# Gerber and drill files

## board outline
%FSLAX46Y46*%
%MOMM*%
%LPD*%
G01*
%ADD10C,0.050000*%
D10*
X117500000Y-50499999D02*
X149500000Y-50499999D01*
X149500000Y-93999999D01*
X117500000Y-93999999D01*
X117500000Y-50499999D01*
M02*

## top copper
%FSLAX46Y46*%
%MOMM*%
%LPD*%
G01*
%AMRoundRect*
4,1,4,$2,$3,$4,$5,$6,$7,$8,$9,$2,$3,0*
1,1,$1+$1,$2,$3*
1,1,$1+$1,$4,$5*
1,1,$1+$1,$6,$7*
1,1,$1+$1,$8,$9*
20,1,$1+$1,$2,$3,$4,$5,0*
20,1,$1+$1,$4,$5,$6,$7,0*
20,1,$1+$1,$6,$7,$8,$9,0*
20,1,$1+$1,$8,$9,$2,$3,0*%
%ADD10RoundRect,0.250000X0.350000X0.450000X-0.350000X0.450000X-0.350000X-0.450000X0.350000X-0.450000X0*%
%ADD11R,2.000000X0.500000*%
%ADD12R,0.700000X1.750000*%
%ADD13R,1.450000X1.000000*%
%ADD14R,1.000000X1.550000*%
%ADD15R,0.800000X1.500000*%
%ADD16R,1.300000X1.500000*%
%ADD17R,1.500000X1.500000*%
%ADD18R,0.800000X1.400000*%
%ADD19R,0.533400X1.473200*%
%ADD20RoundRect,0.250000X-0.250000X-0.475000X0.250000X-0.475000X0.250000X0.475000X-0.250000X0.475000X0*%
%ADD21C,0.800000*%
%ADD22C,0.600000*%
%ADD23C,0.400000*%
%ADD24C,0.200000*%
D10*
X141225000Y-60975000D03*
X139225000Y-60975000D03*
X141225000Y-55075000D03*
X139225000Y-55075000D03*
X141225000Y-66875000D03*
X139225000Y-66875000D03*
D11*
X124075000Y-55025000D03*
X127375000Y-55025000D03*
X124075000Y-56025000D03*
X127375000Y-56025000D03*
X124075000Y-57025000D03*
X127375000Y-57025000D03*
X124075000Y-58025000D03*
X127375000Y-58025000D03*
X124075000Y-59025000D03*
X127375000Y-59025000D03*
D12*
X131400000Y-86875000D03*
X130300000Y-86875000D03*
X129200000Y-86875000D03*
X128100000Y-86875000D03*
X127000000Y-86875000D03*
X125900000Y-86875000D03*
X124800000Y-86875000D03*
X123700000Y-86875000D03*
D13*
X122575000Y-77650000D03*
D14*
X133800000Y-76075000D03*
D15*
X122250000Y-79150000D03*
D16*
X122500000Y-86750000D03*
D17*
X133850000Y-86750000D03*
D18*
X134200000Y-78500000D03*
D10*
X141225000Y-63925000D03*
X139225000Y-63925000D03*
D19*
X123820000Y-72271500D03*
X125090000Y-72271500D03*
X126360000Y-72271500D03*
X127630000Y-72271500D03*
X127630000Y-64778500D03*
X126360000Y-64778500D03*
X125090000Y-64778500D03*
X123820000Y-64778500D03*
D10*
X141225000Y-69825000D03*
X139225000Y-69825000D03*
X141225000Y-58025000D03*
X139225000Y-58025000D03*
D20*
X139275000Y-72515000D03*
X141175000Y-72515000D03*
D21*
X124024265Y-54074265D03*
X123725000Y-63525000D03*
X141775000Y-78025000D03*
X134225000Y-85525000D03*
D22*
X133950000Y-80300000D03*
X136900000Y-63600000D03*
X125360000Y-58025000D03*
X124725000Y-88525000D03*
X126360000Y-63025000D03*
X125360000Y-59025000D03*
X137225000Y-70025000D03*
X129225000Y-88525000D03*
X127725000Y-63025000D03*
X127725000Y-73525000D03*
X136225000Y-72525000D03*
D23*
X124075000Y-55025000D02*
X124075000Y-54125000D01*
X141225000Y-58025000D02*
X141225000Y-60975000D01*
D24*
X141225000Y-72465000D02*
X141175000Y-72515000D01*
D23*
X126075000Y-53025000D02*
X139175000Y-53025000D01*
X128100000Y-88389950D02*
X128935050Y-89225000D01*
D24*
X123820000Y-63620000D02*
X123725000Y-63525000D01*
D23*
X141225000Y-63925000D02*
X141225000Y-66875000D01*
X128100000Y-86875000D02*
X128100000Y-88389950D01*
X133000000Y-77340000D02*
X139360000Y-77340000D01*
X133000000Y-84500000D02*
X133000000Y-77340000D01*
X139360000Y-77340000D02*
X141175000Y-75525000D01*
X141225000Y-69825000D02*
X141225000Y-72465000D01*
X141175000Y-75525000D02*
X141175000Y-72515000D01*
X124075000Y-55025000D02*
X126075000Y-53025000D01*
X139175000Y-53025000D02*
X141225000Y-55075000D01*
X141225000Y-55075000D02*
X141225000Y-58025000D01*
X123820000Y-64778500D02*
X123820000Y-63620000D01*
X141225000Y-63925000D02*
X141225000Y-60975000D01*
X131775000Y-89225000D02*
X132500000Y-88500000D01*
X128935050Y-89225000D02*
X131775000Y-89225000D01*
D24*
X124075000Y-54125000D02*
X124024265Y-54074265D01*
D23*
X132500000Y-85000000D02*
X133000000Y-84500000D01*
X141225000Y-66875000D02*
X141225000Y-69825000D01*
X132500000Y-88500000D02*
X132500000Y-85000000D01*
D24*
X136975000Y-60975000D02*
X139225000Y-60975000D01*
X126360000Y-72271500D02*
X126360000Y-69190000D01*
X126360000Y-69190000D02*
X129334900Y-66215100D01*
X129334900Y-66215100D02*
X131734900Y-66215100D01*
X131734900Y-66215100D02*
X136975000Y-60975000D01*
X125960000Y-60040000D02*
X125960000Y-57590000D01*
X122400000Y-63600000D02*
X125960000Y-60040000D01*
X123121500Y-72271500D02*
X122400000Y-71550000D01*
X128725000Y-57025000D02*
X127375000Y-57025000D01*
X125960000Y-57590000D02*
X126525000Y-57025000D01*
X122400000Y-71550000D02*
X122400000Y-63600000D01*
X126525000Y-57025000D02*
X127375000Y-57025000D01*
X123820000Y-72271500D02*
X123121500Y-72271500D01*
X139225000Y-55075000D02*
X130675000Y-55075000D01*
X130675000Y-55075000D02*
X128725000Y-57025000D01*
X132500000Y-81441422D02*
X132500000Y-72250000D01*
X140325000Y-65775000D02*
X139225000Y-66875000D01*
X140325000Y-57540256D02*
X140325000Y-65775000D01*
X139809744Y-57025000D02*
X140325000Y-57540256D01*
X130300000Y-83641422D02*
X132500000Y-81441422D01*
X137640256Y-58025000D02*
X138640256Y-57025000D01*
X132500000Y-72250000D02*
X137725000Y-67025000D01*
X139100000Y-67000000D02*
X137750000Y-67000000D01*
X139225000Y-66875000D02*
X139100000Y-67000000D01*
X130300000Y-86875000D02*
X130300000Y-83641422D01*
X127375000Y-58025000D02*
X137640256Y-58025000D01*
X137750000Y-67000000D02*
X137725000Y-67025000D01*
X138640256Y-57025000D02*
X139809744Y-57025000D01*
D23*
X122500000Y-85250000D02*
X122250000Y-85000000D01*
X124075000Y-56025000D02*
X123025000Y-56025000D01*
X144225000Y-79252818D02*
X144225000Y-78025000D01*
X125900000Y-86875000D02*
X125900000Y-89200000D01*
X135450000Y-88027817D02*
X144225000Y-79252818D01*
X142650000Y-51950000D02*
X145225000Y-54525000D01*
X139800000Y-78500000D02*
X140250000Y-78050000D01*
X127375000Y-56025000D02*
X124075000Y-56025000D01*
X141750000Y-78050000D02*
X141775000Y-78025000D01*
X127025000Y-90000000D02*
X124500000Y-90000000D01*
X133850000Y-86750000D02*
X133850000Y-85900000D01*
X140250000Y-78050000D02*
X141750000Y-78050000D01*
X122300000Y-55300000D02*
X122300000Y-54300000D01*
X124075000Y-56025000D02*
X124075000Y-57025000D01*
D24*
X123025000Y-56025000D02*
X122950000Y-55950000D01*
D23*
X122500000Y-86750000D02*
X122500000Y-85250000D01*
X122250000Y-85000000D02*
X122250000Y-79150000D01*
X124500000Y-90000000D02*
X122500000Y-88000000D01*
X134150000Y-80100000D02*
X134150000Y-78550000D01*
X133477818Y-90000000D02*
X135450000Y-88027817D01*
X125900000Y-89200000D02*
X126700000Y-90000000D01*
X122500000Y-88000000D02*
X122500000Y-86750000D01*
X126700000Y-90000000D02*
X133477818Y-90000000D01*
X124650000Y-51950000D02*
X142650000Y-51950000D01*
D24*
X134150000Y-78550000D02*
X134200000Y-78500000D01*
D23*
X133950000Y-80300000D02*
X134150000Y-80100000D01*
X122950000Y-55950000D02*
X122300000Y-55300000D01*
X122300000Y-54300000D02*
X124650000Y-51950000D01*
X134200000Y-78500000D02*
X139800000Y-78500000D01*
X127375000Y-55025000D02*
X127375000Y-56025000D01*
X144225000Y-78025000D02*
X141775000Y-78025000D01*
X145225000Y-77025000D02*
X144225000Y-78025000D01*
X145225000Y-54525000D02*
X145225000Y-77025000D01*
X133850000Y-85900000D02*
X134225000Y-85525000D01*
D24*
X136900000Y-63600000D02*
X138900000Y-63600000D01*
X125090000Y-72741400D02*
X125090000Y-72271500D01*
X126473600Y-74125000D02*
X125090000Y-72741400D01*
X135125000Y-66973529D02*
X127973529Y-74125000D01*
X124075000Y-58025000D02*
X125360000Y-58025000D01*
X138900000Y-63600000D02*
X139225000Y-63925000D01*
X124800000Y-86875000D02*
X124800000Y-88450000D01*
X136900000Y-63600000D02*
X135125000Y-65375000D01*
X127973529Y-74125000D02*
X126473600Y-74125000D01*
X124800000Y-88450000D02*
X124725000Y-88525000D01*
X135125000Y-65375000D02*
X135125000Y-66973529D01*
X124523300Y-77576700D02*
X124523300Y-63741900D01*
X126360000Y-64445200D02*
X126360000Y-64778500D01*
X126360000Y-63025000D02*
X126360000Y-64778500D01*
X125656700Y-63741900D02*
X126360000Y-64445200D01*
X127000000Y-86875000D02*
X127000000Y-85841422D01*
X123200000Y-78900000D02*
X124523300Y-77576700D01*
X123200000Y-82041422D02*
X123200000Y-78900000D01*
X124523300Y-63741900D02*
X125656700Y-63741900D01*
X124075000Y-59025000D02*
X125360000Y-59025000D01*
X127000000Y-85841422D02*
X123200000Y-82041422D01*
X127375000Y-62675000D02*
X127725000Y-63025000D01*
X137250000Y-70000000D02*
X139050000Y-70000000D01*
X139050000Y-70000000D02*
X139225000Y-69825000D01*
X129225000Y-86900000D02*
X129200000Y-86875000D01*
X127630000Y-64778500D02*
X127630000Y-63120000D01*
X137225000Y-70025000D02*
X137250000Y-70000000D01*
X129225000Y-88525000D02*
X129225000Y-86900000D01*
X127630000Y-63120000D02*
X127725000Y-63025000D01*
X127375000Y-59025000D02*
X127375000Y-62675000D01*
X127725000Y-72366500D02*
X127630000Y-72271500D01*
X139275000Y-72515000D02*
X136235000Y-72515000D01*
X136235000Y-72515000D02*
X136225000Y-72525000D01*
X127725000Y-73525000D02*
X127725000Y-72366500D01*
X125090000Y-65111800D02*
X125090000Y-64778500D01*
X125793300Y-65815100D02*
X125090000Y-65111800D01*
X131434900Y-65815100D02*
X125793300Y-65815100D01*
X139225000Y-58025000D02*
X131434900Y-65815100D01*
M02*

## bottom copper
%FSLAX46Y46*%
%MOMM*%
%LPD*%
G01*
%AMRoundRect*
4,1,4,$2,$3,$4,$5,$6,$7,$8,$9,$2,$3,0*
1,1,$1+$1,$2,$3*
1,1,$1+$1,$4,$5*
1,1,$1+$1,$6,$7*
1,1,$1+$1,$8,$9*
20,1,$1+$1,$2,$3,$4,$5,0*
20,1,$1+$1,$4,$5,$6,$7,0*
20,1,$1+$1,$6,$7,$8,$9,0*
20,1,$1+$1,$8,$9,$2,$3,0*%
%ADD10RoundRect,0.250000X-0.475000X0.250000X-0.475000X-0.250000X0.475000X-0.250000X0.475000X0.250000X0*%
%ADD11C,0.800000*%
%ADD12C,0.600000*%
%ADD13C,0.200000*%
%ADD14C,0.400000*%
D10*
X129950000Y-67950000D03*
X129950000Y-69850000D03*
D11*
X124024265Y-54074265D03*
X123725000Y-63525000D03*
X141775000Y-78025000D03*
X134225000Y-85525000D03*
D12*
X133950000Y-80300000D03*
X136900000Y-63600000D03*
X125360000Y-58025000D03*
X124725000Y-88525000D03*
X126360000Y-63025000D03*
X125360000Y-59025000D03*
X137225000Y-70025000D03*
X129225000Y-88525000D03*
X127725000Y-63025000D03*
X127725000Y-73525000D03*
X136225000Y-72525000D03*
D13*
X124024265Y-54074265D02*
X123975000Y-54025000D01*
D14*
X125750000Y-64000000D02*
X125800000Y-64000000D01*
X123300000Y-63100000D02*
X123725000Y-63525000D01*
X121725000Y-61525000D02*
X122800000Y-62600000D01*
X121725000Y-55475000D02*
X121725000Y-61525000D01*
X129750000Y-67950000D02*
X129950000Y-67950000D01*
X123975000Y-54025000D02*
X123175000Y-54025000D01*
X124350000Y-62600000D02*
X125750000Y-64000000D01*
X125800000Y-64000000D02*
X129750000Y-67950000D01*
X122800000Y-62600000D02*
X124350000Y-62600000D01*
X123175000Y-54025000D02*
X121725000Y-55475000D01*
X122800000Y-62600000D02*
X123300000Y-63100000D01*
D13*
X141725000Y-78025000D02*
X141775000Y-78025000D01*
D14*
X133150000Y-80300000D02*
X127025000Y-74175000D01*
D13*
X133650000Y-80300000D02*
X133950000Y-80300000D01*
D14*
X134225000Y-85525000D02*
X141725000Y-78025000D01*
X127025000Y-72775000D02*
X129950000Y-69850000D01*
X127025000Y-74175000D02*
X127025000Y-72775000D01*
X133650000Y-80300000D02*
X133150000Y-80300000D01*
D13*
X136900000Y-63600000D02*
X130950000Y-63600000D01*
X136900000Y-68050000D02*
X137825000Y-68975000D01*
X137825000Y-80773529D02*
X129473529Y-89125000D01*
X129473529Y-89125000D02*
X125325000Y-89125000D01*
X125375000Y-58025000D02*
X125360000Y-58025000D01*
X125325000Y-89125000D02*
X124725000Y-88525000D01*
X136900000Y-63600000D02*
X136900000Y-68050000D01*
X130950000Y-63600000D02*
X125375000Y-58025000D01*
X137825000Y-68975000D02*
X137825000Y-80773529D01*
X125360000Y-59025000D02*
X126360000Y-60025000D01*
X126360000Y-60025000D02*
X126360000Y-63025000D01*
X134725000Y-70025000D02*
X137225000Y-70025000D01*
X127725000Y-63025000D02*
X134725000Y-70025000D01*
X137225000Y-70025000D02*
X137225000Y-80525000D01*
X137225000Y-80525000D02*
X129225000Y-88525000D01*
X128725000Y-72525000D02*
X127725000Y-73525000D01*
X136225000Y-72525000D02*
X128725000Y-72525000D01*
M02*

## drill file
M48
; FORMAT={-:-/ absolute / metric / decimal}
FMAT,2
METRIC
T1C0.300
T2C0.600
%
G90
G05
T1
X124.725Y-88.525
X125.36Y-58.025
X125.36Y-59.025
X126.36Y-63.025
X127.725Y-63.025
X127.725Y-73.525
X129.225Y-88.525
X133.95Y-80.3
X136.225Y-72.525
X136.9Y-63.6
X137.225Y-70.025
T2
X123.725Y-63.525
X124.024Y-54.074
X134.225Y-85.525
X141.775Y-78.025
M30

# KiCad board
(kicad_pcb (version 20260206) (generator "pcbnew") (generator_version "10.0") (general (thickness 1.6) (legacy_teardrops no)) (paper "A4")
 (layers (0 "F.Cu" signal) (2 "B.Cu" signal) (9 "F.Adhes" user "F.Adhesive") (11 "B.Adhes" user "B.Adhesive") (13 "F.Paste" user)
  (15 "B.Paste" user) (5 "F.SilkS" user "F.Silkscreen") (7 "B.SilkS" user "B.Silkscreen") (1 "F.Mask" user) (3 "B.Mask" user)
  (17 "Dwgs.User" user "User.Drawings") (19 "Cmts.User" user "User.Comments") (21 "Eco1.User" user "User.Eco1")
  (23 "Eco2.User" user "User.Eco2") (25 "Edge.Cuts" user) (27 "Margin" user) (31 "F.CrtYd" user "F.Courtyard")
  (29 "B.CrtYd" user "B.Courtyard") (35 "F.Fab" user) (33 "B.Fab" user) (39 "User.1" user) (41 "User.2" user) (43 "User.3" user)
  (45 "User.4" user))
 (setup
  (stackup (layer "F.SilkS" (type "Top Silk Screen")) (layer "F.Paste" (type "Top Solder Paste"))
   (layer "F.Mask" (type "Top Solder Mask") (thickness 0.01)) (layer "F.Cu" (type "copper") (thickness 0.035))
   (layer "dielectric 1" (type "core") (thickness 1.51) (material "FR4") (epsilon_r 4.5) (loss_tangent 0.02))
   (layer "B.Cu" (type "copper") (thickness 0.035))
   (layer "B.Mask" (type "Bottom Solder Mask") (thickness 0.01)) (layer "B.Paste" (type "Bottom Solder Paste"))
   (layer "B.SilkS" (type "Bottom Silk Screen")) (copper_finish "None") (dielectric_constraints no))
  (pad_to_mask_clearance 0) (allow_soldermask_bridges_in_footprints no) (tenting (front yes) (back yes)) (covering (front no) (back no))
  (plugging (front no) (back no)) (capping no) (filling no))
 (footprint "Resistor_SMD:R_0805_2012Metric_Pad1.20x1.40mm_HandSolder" (layer "F.Cu") (at 140.225 60.975 180)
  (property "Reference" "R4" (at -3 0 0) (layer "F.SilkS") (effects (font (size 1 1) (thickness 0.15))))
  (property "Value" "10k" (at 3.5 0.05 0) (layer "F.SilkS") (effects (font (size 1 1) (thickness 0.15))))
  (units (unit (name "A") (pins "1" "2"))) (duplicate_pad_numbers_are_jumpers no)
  (pad "1" smd roundrect (at -1 0 180) (size 1.2 1.4) (layers "F.Cu" "F.Mask" "F.Paste") (roundrect_rratio 0.208333) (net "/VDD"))
  (pad "2" smd roundrect (at 1 0 180) (size 1.2 1.4) (layers "F.Cu" "F.Mask" "F.Paste") (roundrect_rratio 0.208333)
   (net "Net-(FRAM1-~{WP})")))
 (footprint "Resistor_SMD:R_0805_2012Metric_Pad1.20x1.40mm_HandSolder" (layer "F.Cu") (at 140.225 55.075 180)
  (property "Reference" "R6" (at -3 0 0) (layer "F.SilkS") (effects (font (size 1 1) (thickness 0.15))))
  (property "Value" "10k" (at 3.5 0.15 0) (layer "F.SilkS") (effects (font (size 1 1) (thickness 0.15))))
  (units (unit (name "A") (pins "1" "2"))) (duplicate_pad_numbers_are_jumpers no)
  (pad "1" smd roundrect (at -1 0 180) (size 1.2 1.4) (layers "F.Cu" "F.Mask" "F.Paste") (roundrect_rratio 0.208333) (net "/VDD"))
  (pad "2" smd roundrect (at 1 0 180) (size 1.2 1.4) (layers "F.Cu" "F.Mask" "F.Paste") (roundrect_rratio 0.208333) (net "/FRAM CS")))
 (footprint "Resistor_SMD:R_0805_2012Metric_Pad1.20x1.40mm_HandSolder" (layer "F.Cu") (at 140.225 66.875 180)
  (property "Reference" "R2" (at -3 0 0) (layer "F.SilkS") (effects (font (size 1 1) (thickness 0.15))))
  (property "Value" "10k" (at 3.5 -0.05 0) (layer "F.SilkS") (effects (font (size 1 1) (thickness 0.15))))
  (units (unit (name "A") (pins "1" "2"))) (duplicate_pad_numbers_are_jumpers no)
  (pad "1" smd roundrect (at -1 0 180) (size 1.2 1.4) (layers "F.Cu" "F.Mask" "F.Paste") (roundrect_rratio 0.208333) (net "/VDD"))
  (pad "2" smd roundrect (at 1 0 180) (size 1.2 1.4) (layers "F.Cu" "F.Mask" "F.Paste") (roundrect_rratio 0.208333) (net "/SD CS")))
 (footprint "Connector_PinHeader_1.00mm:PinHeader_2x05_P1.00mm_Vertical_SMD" (layer "F.Cu") (at 125.725 57.025)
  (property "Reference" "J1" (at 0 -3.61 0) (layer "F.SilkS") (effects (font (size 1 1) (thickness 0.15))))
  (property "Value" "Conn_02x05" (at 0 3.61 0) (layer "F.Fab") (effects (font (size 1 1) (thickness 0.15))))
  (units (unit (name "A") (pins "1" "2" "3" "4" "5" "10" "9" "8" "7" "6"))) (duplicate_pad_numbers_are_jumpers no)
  (pad "1" smd rect (at -1.65 -2) (size 2 0.5) (layers "F.Cu" "F.Mask" "F.Paste") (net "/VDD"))
  (pad "2" smd rect (at 1.65 -2) (size 2 0.5) (layers "F.Cu" "F.Mask" "F.Paste") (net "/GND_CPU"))
  (pad "3" smd rect (at -1.65 -1) (size 2 0.5) (layers "F.Cu" "F.Mask" "F.Paste") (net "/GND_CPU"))
  (pad "4" smd rect (at 1.65 -1) (size 2 0.5) (layers "F.Cu" "F.Mask" "F.Paste") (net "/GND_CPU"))
  (pad "5" smd rect (at -1.65 0) (size 2 0.5) (layers "F.Cu" "F.Mask" "F.Paste") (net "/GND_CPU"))
  (pad "6" smd rect (at 1.65 0) (size 2 0.5) (layers "F.Cu" "F.Mask" "F.Paste") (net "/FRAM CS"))
  (pad "7" smd rect (at -1.65 1) (size 2 0.5) (layers "F.Cu" "F.Mask" "F.Paste") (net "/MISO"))
  (pad "8" smd rect (at 1.65 1) (size 2 0.5) (layers "F.Cu" "F.Mask" "F.Paste") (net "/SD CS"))
  (pad "9" smd rect (at -1.65 2) (size 2 0.5) (layers "F.Cu" "F.Mask" "F.Paste") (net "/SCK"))
  (pad "10" smd rect (at 1.65 2) (size 2 0.5) (layers "F.Cu" "F.Mask" "F.Paste") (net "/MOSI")))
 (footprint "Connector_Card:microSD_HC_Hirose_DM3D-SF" (layer "F.Cu") (at 128.225 81.525)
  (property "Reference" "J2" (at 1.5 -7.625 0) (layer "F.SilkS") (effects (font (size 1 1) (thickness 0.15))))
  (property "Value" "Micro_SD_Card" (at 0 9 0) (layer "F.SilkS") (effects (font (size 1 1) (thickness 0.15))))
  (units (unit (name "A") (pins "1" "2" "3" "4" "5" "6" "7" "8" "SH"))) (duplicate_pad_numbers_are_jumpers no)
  (pad "1" smd rect (at 3.175 5.35) (size 0.7 1.75) (layers "F.Cu" "F.Mask" "F.Paste") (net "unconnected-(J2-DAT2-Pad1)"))
  (pad "2" smd rect (at 2.075 5.35) (size 0.7 1.75) (layers "F.Cu" "F.Mask" "F.Paste") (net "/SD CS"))
  (pad "3" smd rect (at 0.975 5.35) (size 0.7 1.75) (layers "F.Cu" "F.Mask" "F.Paste") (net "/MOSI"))
  (pad "4" smd rect (at -0.125 5.35) (size 0.7 1.75) (layers "F.Cu" "F.Mask" "F.Paste") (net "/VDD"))
  (pad "5" smd rect (at -1.225 5.35) (size 0.7 1.75) (layers "F.Cu" "F.Mask" "F.Paste") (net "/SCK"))
  (pad "6" smd rect (at -2.325 5.35) (size 0.7 1.75) (layers "F.Cu" "F.Mask" "F.Paste") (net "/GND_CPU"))
  (pad "7" smd rect (at -3.425 5.35) (size 0.7 1.75) (layers "F.Cu" "F.Mask" "F.Paste") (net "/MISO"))
  (pad "8" smd rect (at -4.525 5.35) (size 0.7 1.75) (layers "F.Cu" "F.Mask" "F.Paste") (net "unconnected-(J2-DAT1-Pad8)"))
  (pad "9" smd rect (at -5.65 -3.875) (size 1.45 1) (layers "F.Cu" "F.Mask" "F.Paste"))
  (pad "10" smd rect (at 5.575 -5.45) (size 1 1.55) (layers "F.Cu" "F.Mask" "F.Paste"))
  (pad "SH" smd rect (at -5.975 -2.375) (size 0.8 1.5) (layers "F.Cu" "F.Mask" "F.Paste") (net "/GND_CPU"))
  (pad "SH" smd rect (at -5.725 5.225) (size 1.3 1.5) (layers "F.Cu" "F.Mask" "F.Paste") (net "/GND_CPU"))
  (pad "SH" smd rect (at 5.625 5.225) (size 1.5 1.5) (layers "F.Cu" "F.Mask" "F.Paste") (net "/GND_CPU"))
  (pad "SH" smd rect (at 5.975 -3.025) (size 0.8 1.4) (layers "F.Cu" "F.Mask" "F.Paste") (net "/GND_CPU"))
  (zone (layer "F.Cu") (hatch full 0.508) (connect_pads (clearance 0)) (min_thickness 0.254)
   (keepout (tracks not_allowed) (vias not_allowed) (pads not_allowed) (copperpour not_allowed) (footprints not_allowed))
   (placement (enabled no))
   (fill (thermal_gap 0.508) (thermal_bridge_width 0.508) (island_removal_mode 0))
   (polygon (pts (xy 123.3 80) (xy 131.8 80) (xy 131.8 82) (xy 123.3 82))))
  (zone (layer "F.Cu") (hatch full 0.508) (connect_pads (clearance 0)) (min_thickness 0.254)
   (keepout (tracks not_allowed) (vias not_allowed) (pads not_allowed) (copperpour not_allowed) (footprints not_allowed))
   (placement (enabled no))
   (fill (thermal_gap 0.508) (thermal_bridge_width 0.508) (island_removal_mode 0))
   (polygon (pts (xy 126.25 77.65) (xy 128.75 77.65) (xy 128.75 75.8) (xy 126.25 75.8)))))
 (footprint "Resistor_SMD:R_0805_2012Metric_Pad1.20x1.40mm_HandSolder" (layer "F.Cu") (at 140.225 63.925 180)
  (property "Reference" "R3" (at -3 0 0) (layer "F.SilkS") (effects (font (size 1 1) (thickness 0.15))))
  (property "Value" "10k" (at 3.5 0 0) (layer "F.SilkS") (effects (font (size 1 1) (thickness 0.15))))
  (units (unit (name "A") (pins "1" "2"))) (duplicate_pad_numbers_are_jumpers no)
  (pad "1" smd roundrect (at -1 0 180) (size 1.2 1.4) (layers "F.Cu" "F.Mask" "F.Paste") (roundrect_rratio 0.208333) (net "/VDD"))
  (pad "2" smd roundrect (at 1 0 180) (size 1.2 1.4) (layers "F.Cu" "F.Mask" "F.Paste") (roundrect_rratio 0.208333) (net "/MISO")))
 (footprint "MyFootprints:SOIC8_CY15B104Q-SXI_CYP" (layer "F.Cu") (at 125.725 68.525 90)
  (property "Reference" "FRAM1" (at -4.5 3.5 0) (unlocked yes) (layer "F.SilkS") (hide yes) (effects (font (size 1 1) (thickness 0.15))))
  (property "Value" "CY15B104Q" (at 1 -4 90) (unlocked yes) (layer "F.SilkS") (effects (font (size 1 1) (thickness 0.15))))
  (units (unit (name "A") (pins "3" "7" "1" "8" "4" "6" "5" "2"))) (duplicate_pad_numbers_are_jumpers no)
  (pad "1" smd rect (at -3.7465 -1.905 90) (size 1.4732 0.5334) (layers "F.Cu" "F.Mask" "F.Paste") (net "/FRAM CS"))
  (pad "2" smd rect (at -3.7465 -0.635 90) (size 1.4732 0.5334) (layers "F.Cu" "F.Mask" "F.Paste") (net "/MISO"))
  (pad "3" smd rect (at -3.7465 0.635 90) (size 1.4732 0.5334) (layers "F.Cu" "F.Mask" "F.Paste") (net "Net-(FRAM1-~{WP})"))
  (pad "4" smd rect (at -3.7465 1.905 90) (size 1.4732 0.5334) (layers "F.Cu" "F.Mask" "F.Paste") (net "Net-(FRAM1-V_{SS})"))
  (pad "5" smd rect (at 3.7465 1.905 90) (size 1.4732 0.5334) (layers "F.Cu" "F.Mask" "F.Paste") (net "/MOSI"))
  (pad "6" smd rect (at 3.7465 0.635 90) (size 1.4732 0.5334) (layers "F.Cu" "F.Mask" "F.Paste") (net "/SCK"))
  (pad "7" smd rect (at 3.7465 -0.635 90) (size 1.4732 0.5334) (layers "F.Cu" "F.Mask" "F.Paste") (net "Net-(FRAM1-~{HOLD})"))
  (pad "8" smd rect (at 3.7465 -1.905 90) (size 1.4732 0.5334) (layers "F.Cu" "F.Mask" "F.Paste") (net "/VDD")))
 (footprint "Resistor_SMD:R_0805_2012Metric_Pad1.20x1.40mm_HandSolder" (layer "F.Cu") (at 140.225 69.825 180)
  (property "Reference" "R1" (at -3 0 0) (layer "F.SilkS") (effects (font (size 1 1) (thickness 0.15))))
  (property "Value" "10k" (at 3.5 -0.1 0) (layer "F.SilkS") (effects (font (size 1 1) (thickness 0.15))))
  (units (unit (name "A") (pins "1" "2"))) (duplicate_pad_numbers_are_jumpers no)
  (pad "1" smd roundrect (at -1 0 180) (size 1.2 1.4) (layers "F.Cu" "F.Mask" "F.Paste") (roundrect_rratio 0.208333) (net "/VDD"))
  (pad "2" smd roundrect (at 1 0 180) (size 1.2 1.4) (layers "F.Cu" "F.Mask" "F.Paste") (roundrect_rratio 0.208333) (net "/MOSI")))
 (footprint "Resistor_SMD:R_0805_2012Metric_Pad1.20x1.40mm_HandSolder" (layer "F.Cu") (at 140.225 58.025 180)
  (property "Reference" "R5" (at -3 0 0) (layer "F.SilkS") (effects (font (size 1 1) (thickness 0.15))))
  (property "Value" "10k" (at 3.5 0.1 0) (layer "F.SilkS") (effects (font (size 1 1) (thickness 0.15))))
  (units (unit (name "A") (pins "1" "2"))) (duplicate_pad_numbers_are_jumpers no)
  (pad "1" smd roundrect (at -1 0 180) (size 1.2 1.4) (layers "F.Cu" "F.Mask" "F.Paste") (roundrect_rratio 0.208333) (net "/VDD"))
  (pad "2" smd roundrect (at 1 0 180) (size 1.2 1.4) (layers "F.Cu" "F.Mask" "F.Paste") (roundrect_rratio 0.208333)
   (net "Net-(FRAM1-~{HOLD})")))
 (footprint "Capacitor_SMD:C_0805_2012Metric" (layer "F.Cu") (at 140.225 72.515)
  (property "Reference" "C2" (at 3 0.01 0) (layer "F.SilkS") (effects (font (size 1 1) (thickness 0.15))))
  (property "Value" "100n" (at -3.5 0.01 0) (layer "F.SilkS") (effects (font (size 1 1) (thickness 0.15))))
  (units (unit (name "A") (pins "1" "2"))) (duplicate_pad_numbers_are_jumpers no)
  (pad "1" smd roundrect (at -0.95 0) (size 1 1.45) (layers "F.Cu" "F.Mask" "F.Paste") (roundrect_rratio 0.25) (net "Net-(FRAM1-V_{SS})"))
  (pad "2" smd roundrect (at 0.95 0) (size 1 1.45) (layers "F.Cu" "F.Mask" "F.Paste") (roundrect_rratio 0.25) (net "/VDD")))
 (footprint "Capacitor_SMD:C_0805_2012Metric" (layer "B.Cu") (at 129.95 68.9 -90)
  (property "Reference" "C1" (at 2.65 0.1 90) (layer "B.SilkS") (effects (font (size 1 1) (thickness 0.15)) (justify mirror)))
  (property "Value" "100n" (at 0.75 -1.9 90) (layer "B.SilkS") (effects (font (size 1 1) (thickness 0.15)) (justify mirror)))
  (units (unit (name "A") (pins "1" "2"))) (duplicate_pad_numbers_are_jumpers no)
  (pad "1" smd roundrect (at -0.95 0 270) (size 1 1.45) (layers "B.Cu" "B.Mask" "B.Paste") (roundrect_rratio 0.25) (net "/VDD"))
  (pad "2" smd roundrect (at 0.95 0 270) (size 1 1.45) (layers "B.Cu" "B.Mask" "B.Paste") (roundrect_rratio 0.25) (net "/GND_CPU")))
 (gr_rect (start 117.5 50.499999) (end 149.5 93.999999) (stroke (width 0.05) (type solid)) (fill no) (layer "Edge.Cuts"))
 (segment (start 124.075 55.025) (end 124.075 54.125) (width 0.4) (layer "F.Cu") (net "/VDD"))
 (segment (start 141.225 58.025) (end 141.225 60.975) (width 0.4) (layer "F.Cu") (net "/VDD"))
 (segment (start 141.225 72.465) (end 141.175 72.515) (width 0.2) (layer "F.Cu") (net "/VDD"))
 (segment (start 126.075 53.025) (end 139.175 53.025) (width 0.4) (layer "F.Cu") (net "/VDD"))
 (segment (start 128.1 88.38995) (end 128.93505 89.225) (width 0.4) (layer "F.Cu") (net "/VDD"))
 (segment (start 123.82 63.62) (end 123.725 63.525) (width 0.2) (layer "F.Cu") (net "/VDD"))
 (segment (start 141.225 63.925) (end 141.225 66.875) (width 0.4) (layer "F.Cu") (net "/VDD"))
 (segment (start 128.1 86.875) (end 128.1 88.38995) (width 0.4) (layer "F.Cu") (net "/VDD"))
 (segment (start 133 77.34) (end 139.36 77.34) (width 0.4) (layer "F.Cu") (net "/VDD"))
 (segment (start 133 84.5) (end 133 77.34) (width 0.4) (layer "F.Cu") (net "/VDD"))
 (segment (start 139.36 77.34) (end 141.175 75.525) (width 0.4) (layer "F.Cu") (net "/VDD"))
 (segment (start 141.225 69.825) (end 141.225 72.465) (width 0.4) (layer "F.Cu") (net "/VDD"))
 (segment (start 141.175 75.525) (end 141.175 72.515) (width 0.4) (layer "F.Cu") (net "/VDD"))
 (segment (start 124.075 55.025) (end 126.075 53.025) (width 0.4) (layer "F.Cu") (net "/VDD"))
 (segment (start 139.175 53.025) (end 141.225 55.075) (width 0.4) (layer "F.Cu") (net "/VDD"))
 (segment (start 141.225 55.075) (end 141.225 58.025) (width 0.4) (layer "F.Cu") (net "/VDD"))
 (segment (start 123.82 64.7785) (end 123.82 63.62) (width 0.4) (layer "F.Cu") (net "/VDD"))
 (segment (start 141.225 63.925) (end 141.225 60.975) (width 0.4) (layer "F.Cu") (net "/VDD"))
 (segment (start 131.775 89.225) (end 132.5 88.5) (width 0.4) (layer "F.Cu") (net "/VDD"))
 (segment (start 128.93505 89.225) (end 131.775 89.225) (width 0.4) (layer "F.Cu") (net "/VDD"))
 (segment (start 124.075 54.125) (end 124.024265 54.074265) (width 0.2) (layer "F.Cu") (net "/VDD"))
 (segment (start 132.5 85) (end 133 84.5) (width 0.4) (layer "F.Cu") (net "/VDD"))
 (segment (start 141.225 66.875) (end 141.225 69.825) (width 0.4) (layer "F.Cu") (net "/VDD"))
 (segment (start 132.5 88.5) (end 132.5 85) (width 0.4) (layer "F.Cu") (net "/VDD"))
 (via (at 124.024265 54.074265) (size 0.8) (drill 0.6) (layers "F.Cu" "B.Cu") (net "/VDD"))
 (via (at 123.725 63.525) (size 0.8) (drill 0.6) (layers "F.Cu" "B.Cu") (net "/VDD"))
 (segment (start 124.024265 54.074265) (end 123.975 54.025) (width 0.2) (layer "B.Cu") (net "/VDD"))
 (segment (start 125.75 64) (end 125.8 64) (width 0.4) (layer "B.Cu") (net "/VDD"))
 (segment (start 123.3 63.1) (end 123.725 63.525) (width 0.4) (layer "B.Cu") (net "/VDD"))
 (segment (start 121.725 61.525) (end 122.8 62.6) (width 0.4) (layer "B.Cu") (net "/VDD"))
 (segment (start 121.725 55.475) (end 121.725 61.525) (width 0.4) (layer "B.Cu") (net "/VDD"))
 (segment (start 129.75 67.95) (end 129.95 67.95) (width 0.4) (layer "B.Cu") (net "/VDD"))
 (segment (start 123.975 54.025) (end 123.175 54.025) (width 0.4) (layer "B.Cu") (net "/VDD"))
 (segment (start 124.35 62.6) (end 125.75 64) (width 0.4) (layer "B.Cu") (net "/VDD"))
 (segment (start 125.8 64) (end 129.75 67.95) (width 0.4) (layer "B.Cu") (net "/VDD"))
 (segment (start 122.8 62.6) (end 124.35 62.6) (width 0.4) (layer "B.Cu") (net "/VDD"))
 (segment (start 123.175 54.025) (end 121.725 55.475) (width 0.4) (layer "B.Cu") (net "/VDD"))
 (segment (start 122.8 62.6) (end 123.3 63.1) (width 0.4) (layer "B.Cu") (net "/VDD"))
 (segment (start 136.975 60.975) (end 139.225 60.975) (width 0.2) (layer "F.Cu") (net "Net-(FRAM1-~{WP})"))
 (segment (start 126.36 72.2715) (end 126.36 69.19) (width 0.2) (layer "F.Cu") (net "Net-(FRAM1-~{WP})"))
 (segment (start 126.36 69.19) (end 129.3349 66.2151) (width 0.2) (layer "F.Cu") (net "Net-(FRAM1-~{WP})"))
 (segment (start 129.3349 66.2151) (end 131.7349 66.2151) (width 0.2) (layer "F.Cu") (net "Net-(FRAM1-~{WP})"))
 (segment (start 131.7349 66.2151) (end 136.975 60.975) (width 0.2) (layer "F.Cu") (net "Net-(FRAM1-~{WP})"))
 (segment (start 125.96 60.04) (end 125.96 57.59) (width 0.2) (layer "F.Cu") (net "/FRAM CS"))
 (segment (start 122.4 63.6) (end 125.96 60.04) (width 0.2) (layer "F.Cu") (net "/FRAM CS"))
 (segment (start 123.1215 72.2715) (end 122.4 71.55) (width 0.2) (layer "F.Cu") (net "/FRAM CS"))
 (segment (start 128.725 57.025) (end 127.375 57.025) (width 0.2) (layer "F.Cu") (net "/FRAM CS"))
 (segment (start 125.96 57.59) (end 126.525 57.025) (width 0.2) (layer "F.Cu") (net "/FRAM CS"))
 (segment (start 122.4 71.55) (end 122.4 63.6) (width 0.2) (layer "F.Cu") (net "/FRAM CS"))
 (segment (start 126.525 57.025) (end 127.375 57.025) (width 0.2) (layer "F.Cu") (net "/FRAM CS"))
 (segment (start 123.82 72.2715) (end 123.1215 72.2715) (width 0.2) (layer "F.Cu") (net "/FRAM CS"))
 (segment (start 139.225 55.075) (end 130.675 55.075) (width 0.2) (layer "F.Cu") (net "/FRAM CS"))
 (segment (start 130.675 55.075) (end 128.725 57.025) (width 0.2) (layer "F.Cu") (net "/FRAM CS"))
 (segment (start 132.5 81.441422) (end 132.5 72.25) (width 0.2) (layer "F.Cu") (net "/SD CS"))
 (segment (start 140.325 65.775) (end 139.225 66.875) (width 0.2) (layer "F.Cu") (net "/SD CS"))
 (segment (start 140.325 57.540256) (end 140.325 65.775) (width 0.2) (layer "F.Cu") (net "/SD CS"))
 (segment (start 139.809744 57.025) (end 140.325 57.540256) (width 0.2) (layer "F.Cu") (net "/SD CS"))
 (segment (start 130.3 83.641422) (end 132.5 81.441422) (width 0.2) (layer "F.Cu") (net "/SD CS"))
 (segment (start 137.640256 58.025) (end 138.640256 57.025) (width 0.2) (layer "F.Cu") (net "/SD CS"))
 (segment (start 132.5 72.25) (end 137.725 67.025) (width 0.2) (layer "F.Cu") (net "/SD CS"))
 (segment (start 139.1 67) (end 137.75 67) (width 0.2) (layer "F.Cu") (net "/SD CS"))
 (segment (start 139.225 66.875) (end 139.1 67) (width 0.2) (layer "F.Cu") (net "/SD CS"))
 (segment (start 130.3 86.875) (end 130.3 83.641422) (width 0.2) (layer "F.Cu") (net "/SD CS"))
 (segment (start 127.375 58.025) (end 137.640256 58.025) (width 0.2) (layer "F.Cu") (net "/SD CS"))
 (segment (start 137.75 67) (end 137.725 67.025) (width 0.2) (layer "F.Cu") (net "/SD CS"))
 (segment (start 138.640256 57.025) (end 139.809744 57.025) (width 0.2) (layer "F.Cu") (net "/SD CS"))
 (segment (start 122.5 85.25) (end 122.25 85) (width 0.4) (layer "F.Cu") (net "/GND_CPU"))
 (segment (start 124.075 56.025) (end 123.025 56.025) (width 0.4) (layer "F.Cu") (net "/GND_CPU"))
 (segment (start 144.225 79.252818) (end 144.225 78.025) (width 0.4) (layer "F.Cu") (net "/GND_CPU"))
 (segment (start 125.9 86.875) (end 125.9 89.2) (width 0.4) (layer "F.Cu") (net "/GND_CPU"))
 (segment (start 135.45 88.027817) (end 144.225 79.252818) (width 0.4) (layer "F.Cu") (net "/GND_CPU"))
 (segment (start 142.65 51.95) (end 145.225 54.525) (width 0.4) (layer "F.Cu") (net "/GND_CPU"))
 (segment (start 139.8 78.5) (end 140.25 78.05) (width 0.4) (layer "F.Cu") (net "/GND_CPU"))
 (segment (start 127.375 56.025) (end 124.075 56.025) (width 0.4) (layer "F.Cu") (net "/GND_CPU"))
 (segment (start 141.75 78.05) (end 141.775 78.025) (width 0.4) (layer "F.Cu") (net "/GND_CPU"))
 (segment (start 127.025 90) (end 124.5 90) (width 0.4) (layer "F.Cu") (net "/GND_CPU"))
 (segment (start 133.85 86.75) (end 133.85 85.9) (width 0.4) (layer "F.Cu") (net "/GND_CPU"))
 (segment (start 140.25 78.05) (end 141.75 78.05) (width 0.4) (layer "F.Cu") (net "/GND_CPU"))
 (segment (start 122.3 55.3) (end 122.3 54.3) (width 0.4) (layer "F.Cu") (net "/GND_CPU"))
 (segment (start 124.075 56.025) (end 124.075 57.025) (width 0.4) (layer "F.Cu") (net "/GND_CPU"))
 (segment (start 123.025 56.025) (end 122.95 55.95) (width 0.2) (layer "F.Cu") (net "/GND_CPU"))
 (segment (start 122.5 86.75) (end 122.5 85.25) (width 0.4) (layer "F.Cu") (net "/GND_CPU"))
 (segment (start 122.25 85) (end 122.25 79.15) (width 0.4) (layer "F.Cu") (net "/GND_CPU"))
 (segment (start 124.5 90) (end 122.5 88) (width 0.4) (layer "F.Cu") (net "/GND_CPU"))
 (segment (start 134.15 80.1) (end 134.15 78.55) (width 0.4) (layer "F.Cu") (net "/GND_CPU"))
 (segment (start 133.477818 90) (end 135.45 88.027817) (width 0.4) (layer "F.Cu") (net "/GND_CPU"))
 (segment (start 125.9 89.2) (end 126.7 90) (width 0.4) (layer "F.Cu") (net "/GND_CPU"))
 (segment (start 122.5 88) (end 122.5 86.75) (width 0.4) (layer "F.Cu") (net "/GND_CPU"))
 (segment (start 126.7 90) (end 133.477818 90) (width 0.4) (layer "F.Cu") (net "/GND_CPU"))
 (segment (start 124.65 51.95) (end 142.65 51.95) (width 0.4) (layer "F.Cu") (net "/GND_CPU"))
 (segment (start 134.15 78.55) (end 134.2 78.5) (width 0.2) (layer "F.Cu") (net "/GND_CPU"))
 (segment (start 133.95 80.3) (end 134.15 80.1) (width 0.4) (layer "F.Cu") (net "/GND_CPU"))
 (segment (start 122.95 55.95) (end 122.3 55.3) (width 0.4) (layer "F.Cu") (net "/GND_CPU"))
 (segment (start 122.3 54.3) (end 124.65 51.95) (width 0.4) (layer "F.Cu") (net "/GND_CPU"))
 (segment (start 134.2 78.5) (end 139.8 78.5) (width 0.4) (layer "F.Cu") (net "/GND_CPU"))
 (segment (start 127.375 55.025) (end 127.375 56.025) (width 0.4) (layer "F.Cu") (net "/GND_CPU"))
 (segment (start 144.225 78.025) (end 141.775 78.025) (width 0.4) (layer "F.Cu") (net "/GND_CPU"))
 (segment (start 145.225 77.025) (end 144.225 78.025) (width 0.4) (layer "F.Cu") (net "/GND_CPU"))
 (segment (start 145.225 54.525) (end 145.225 77.025) (width 0.4) (layer "F.Cu") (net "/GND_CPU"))
 (segment (start 133.85 85.9) (end 134.225 85.525) (width 0.4) (layer "F.Cu") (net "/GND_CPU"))
 (via (at 141.775 78.025) (size 0.8) (drill 0.6) (layers "F.Cu" "B.Cu") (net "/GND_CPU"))
 (via (at 134.225 85.525) (size 0.8) (drill 0.6) (layers "F.Cu" "B.Cu") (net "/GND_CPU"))
 (via (at 133.95 80.3) (size 0.6) (drill 0.3) (layers "F.Cu" "B.Cu") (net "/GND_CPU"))
 (segment (start 141.725 78.025) (end 141.775 78.025) (width 0.2) (layer "B.Cu") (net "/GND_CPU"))
 (segment (start 133.15 80.3) (end 127.025 74.175) (width 0.4) (layer "B.Cu") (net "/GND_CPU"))
 (segment (start 133.65 80.3) (end 133.95 80.3) (width 0.2) (layer "B.Cu") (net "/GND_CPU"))
 (segment (start 134.225 85.525) (end 141.725 78.025) (width 0.4) (layer "B.Cu") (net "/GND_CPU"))
 (segment (start 127.025 72.775) (end 129.95 69.85) (width 0.4) (layer "B.Cu") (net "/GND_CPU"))
 (segment (start 127.025 74.175) (end 127.025 72.775) (width 0.4) (layer "B.Cu") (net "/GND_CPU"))
 (segment (start 133.65 80.3) (end 133.15 80.3) (width 0.4) (layer "B.Cu") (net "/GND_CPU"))
 (segment (start 136.9 63.6) (end 138.9 63.6) (width 0.2) (layer "F.Cu") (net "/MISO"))
 (segment (start 125.09 72.7414) (end 125.09 72.2715) (width 0.2) (layer "F.Cu") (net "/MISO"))
 (segment (start 126.4736 74.125) (end 125.09 72.7414) (width 0.2) (layer "F.Cu") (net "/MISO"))
 (segment (start 135.125 66.973529) (end 127.973529 74.125) (width 0.2) (layer "F.Cu") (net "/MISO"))
 (segment (start 124.075 58.025) (end 125.36 58.025) (width 0.2) (layer "F.Cu") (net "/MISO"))
 (segment (start 138.9 63.6) (end 139.225 63.925) (width 0.2) (layer "F.Cu") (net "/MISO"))
 (segment (start 124.8 86.875) (end 124.8 88.45) (width 0.2) (layer "F.Cu") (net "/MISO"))
 (segment (start 136.9 63.6) (end 135.125 65.375) (width 0.2) (layer "F.Cu") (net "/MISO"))
 (segment (start 127.973529 74.125) (end 126.4736 74.125) (width 0.2) (layer "F.Cu") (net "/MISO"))
 (segment (start 124.8 88.45) (end 124.725 88.525) (width 0.2) (layer "F.Cu") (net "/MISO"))
 (segment (start 135.125 65.375) (end 135.125 66.973529) (width 0.2) (layer "F.Cu") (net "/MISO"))
 (via (at 136.9 63.6) (size 0.6) (drill 0.3) (layers "F.Cu" "B.Cu") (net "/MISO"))
 (via (at 125.36 58.025) (size 0.6) (drill 0.3) (layers "F.Cu" "B.Cu") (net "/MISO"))
 (via (at 124.725 88.525) (size 0.6) (drill 0.3) (layers "F.Cu" "B.Cu") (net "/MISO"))
 (segment (start 136.9 63.6) (end 130.95 63.6) (width 0.2) (layer "B.Cu") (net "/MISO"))
 (segment (start 136.9 68.05) (end 137.825 68.975) (width 0.2) (layer "B.Cu") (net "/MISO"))
 (segment (start 137.825 80.773529) (end 129.473529 89.125) (width 0.2) (layer "B.Cu") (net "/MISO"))
 (segment (start 129.473529 89.125) (end 125.325 89.125) (width 0.2) (layer "B.Cu") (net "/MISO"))
 (segment (start 125.375 58.025) (end 125.36 58.025) (width 0.2) (layer "B.Cu") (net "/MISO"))
 (segment (start 125.325 89.125) (end 124.725 88.525) (width 0.2) (layer "B.Cu") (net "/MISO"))
 (segment (start 136.9 63.6) (end 136.9 68.05) (width 0.2) (layer "B.Cu") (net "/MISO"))
 (segment (start 130.95 63.6) (end 125.375 58.025) (width 0.2) (layer "B.Cu") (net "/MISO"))
 (segment (start 137.825 68.975) (end 137.825 80.773529) (width 0.2) (layer "B.Cu") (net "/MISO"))
 (segment (start 124.5233 77.5767) (end 124.5233 63.7419) (width 0.2) (layer "F.Cu") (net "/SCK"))
 (segment (start 126.36 64.4452) (end 126.36 64.7785) (width 0.2) (layer "F.Cu") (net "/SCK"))
 (segment (start 126.36 63.025) (end 126.36 64.7785) (width 0.2) (layer "F.Cu") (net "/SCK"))
 (segment (start 125.6567 63.7419) (end 126.36 64.4452) (width 0.2) (layer "F.Cu") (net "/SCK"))
 (segment (start 127 86.875) (end 127 85.841422) (width 0.2) (layer "F.Cu") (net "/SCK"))
 (segment (start 123.2 78.9) (end 124.5233 77.5767) (width 0.2) (layer "F.Cu") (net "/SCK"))
 (segment (start 123.2 82.041422) (end 123.2 78.9) (width 0.2) (layer "F.Cu") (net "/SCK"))
 (segment (start 124.5233 63.7419) (end 125.6567 63.7419) (width 0.2) (layer "F.Cu") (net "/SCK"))
 (segment (start 124.075 59.025) (end 125.36 59.025) (width 0.2) (layer "F.Cu") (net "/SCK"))
 (segment (start 127 85.841422) (end 123.2 82.041422) (width 0.2) (layer "F.Cu") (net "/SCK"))
 (via (at 126.36 63.025) (size 0.6) (drill 0.3) (layers "F.Cu" "B.Cu") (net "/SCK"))
 (via (at 125.36 59.025) (size 0.6) (drill 0.3) (layers "F.Cu" "B.Cu") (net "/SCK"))
 (segment (start 125.36 59.025) (end 126.36 60.025) (width 0.2) (layer "B.Cu") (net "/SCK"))
 (segment (start 126.36 60.025) (end 126.36 63.025) (width 0.2) (layer "B.Cu") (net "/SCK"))
 (segment (start 127.375 62.675) (end 127.725 63.025) (width 0.2) (layer "F.Cu") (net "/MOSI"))
 (segment (start 137.25 70) (end 139.05 70) (width 0.2) (layer "F.Cu") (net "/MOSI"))
 (segment (start 139.05 70) (end 139.225 69.825) (width 0.2) (layer "F.Cu") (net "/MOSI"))
 (segment (start 129.225 86.9) (end 129.2 86.875) (width 0.2) (layer "F.Cu") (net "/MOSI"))
 (segment (start 127.63 64.7785) (end 127.63 63.12) (width 0.2) (layer "F.Cu") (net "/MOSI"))
 (segment (start 137.225 70.025) (end 137.25 70) (width 0.2) (layer "F.Cu") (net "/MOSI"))
 (segment (start 129.225 88.525) (end 129.225 86.9) (width 0.2) (layer "F.Cu") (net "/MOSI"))
 (segment (start 127.63 63.12) (end 127.725 63.025) (width 0.2) (layer "F.Cu") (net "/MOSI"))
 (segment (start 127.375 59.025) (end 127.375 62.675) (width 0.2) (layer "F.Cu") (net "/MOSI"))
 (via (at 137.225 70.025) (size 0.6) (drill 0.3) (layers "F.Cu" "B.Cu") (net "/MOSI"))
 (via (at 129.225 88.525) (size 0.6) (drill 0.3) (layers "F.Cu" "B.Cu") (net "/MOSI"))
 (via (at 127.725 63.025) (size 0.6) (drill 0.3) (layers "F.Cu" "B.Cu") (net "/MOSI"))
 (segment (start 134.725 70.025) (end 137.225 70.025) (width 0.2) (layer "B.Cu") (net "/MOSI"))
 (segment (start 127.725 63.025) (end 134.725 70.025) (width 0.2) (layer "B.Cu") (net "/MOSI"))
 (segment (start 137.225 70.025) (end 137.225 80.525) (width 0.2) (layer "B.Cu") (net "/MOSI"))
 (segment (start 137.225 80.525) (end 129.225 88.525) (width 0.2) (layer "B.Cu") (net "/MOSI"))
 (segment (start 127.725 72.3665) (end 127.63 72.2715) (width 0.2) (layer "F.Cu") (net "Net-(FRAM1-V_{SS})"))
 (segment (start 139.275 72.515) (end 136.235 72.515) (width 0.2) (layer "F.Cu") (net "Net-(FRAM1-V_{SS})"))
 (segment (start 136.235 72.515) (end 136.225 72.525) (width 0.2) (layer "F.Cu") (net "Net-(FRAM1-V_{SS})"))
 (segment (start 127.725 73.525) (end 127.725 72.3665) (width 0.2) (layer "F.Cu") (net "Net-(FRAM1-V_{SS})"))
 (via (at 127.725 73.525) (size 0.6) (drill 0.3) (layers "F.Cu" "B.Cu") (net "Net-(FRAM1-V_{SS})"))
 (via (at 136.225 72.525) (size 0.6) (drill 0.3) (layers "F.Cu" "B.Cu") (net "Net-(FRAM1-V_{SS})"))
 (segment (start 128.725 72.525) (end 127.725 73.525) (width 0.2) (layer "B.Cu") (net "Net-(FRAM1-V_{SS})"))
 (segment (start 136.225 72.525) (end 128.725 72.525) (width 0.2) (layer "B.Cu") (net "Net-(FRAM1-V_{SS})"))
 (segment (start 125.09 65.1118) (end 125.09 64.7785) (width 0.2) (layer "F.Cu") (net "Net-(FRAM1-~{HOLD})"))
 (segment (start 125.7933 65.8151) (end 125.09 65.1118) (width 0.2) (layer "F.Cu") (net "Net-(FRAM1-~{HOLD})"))
 (segment (start 131.4349 65.8151) (end 125.7933 65.8151) (width 0.2) (layer "F.Cu") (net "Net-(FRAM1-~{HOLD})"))
 (segment (start 139.225 58.025) (end 131.4349 65.8151) (width 0.2) (layer "F.Cu") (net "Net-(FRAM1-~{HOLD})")))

